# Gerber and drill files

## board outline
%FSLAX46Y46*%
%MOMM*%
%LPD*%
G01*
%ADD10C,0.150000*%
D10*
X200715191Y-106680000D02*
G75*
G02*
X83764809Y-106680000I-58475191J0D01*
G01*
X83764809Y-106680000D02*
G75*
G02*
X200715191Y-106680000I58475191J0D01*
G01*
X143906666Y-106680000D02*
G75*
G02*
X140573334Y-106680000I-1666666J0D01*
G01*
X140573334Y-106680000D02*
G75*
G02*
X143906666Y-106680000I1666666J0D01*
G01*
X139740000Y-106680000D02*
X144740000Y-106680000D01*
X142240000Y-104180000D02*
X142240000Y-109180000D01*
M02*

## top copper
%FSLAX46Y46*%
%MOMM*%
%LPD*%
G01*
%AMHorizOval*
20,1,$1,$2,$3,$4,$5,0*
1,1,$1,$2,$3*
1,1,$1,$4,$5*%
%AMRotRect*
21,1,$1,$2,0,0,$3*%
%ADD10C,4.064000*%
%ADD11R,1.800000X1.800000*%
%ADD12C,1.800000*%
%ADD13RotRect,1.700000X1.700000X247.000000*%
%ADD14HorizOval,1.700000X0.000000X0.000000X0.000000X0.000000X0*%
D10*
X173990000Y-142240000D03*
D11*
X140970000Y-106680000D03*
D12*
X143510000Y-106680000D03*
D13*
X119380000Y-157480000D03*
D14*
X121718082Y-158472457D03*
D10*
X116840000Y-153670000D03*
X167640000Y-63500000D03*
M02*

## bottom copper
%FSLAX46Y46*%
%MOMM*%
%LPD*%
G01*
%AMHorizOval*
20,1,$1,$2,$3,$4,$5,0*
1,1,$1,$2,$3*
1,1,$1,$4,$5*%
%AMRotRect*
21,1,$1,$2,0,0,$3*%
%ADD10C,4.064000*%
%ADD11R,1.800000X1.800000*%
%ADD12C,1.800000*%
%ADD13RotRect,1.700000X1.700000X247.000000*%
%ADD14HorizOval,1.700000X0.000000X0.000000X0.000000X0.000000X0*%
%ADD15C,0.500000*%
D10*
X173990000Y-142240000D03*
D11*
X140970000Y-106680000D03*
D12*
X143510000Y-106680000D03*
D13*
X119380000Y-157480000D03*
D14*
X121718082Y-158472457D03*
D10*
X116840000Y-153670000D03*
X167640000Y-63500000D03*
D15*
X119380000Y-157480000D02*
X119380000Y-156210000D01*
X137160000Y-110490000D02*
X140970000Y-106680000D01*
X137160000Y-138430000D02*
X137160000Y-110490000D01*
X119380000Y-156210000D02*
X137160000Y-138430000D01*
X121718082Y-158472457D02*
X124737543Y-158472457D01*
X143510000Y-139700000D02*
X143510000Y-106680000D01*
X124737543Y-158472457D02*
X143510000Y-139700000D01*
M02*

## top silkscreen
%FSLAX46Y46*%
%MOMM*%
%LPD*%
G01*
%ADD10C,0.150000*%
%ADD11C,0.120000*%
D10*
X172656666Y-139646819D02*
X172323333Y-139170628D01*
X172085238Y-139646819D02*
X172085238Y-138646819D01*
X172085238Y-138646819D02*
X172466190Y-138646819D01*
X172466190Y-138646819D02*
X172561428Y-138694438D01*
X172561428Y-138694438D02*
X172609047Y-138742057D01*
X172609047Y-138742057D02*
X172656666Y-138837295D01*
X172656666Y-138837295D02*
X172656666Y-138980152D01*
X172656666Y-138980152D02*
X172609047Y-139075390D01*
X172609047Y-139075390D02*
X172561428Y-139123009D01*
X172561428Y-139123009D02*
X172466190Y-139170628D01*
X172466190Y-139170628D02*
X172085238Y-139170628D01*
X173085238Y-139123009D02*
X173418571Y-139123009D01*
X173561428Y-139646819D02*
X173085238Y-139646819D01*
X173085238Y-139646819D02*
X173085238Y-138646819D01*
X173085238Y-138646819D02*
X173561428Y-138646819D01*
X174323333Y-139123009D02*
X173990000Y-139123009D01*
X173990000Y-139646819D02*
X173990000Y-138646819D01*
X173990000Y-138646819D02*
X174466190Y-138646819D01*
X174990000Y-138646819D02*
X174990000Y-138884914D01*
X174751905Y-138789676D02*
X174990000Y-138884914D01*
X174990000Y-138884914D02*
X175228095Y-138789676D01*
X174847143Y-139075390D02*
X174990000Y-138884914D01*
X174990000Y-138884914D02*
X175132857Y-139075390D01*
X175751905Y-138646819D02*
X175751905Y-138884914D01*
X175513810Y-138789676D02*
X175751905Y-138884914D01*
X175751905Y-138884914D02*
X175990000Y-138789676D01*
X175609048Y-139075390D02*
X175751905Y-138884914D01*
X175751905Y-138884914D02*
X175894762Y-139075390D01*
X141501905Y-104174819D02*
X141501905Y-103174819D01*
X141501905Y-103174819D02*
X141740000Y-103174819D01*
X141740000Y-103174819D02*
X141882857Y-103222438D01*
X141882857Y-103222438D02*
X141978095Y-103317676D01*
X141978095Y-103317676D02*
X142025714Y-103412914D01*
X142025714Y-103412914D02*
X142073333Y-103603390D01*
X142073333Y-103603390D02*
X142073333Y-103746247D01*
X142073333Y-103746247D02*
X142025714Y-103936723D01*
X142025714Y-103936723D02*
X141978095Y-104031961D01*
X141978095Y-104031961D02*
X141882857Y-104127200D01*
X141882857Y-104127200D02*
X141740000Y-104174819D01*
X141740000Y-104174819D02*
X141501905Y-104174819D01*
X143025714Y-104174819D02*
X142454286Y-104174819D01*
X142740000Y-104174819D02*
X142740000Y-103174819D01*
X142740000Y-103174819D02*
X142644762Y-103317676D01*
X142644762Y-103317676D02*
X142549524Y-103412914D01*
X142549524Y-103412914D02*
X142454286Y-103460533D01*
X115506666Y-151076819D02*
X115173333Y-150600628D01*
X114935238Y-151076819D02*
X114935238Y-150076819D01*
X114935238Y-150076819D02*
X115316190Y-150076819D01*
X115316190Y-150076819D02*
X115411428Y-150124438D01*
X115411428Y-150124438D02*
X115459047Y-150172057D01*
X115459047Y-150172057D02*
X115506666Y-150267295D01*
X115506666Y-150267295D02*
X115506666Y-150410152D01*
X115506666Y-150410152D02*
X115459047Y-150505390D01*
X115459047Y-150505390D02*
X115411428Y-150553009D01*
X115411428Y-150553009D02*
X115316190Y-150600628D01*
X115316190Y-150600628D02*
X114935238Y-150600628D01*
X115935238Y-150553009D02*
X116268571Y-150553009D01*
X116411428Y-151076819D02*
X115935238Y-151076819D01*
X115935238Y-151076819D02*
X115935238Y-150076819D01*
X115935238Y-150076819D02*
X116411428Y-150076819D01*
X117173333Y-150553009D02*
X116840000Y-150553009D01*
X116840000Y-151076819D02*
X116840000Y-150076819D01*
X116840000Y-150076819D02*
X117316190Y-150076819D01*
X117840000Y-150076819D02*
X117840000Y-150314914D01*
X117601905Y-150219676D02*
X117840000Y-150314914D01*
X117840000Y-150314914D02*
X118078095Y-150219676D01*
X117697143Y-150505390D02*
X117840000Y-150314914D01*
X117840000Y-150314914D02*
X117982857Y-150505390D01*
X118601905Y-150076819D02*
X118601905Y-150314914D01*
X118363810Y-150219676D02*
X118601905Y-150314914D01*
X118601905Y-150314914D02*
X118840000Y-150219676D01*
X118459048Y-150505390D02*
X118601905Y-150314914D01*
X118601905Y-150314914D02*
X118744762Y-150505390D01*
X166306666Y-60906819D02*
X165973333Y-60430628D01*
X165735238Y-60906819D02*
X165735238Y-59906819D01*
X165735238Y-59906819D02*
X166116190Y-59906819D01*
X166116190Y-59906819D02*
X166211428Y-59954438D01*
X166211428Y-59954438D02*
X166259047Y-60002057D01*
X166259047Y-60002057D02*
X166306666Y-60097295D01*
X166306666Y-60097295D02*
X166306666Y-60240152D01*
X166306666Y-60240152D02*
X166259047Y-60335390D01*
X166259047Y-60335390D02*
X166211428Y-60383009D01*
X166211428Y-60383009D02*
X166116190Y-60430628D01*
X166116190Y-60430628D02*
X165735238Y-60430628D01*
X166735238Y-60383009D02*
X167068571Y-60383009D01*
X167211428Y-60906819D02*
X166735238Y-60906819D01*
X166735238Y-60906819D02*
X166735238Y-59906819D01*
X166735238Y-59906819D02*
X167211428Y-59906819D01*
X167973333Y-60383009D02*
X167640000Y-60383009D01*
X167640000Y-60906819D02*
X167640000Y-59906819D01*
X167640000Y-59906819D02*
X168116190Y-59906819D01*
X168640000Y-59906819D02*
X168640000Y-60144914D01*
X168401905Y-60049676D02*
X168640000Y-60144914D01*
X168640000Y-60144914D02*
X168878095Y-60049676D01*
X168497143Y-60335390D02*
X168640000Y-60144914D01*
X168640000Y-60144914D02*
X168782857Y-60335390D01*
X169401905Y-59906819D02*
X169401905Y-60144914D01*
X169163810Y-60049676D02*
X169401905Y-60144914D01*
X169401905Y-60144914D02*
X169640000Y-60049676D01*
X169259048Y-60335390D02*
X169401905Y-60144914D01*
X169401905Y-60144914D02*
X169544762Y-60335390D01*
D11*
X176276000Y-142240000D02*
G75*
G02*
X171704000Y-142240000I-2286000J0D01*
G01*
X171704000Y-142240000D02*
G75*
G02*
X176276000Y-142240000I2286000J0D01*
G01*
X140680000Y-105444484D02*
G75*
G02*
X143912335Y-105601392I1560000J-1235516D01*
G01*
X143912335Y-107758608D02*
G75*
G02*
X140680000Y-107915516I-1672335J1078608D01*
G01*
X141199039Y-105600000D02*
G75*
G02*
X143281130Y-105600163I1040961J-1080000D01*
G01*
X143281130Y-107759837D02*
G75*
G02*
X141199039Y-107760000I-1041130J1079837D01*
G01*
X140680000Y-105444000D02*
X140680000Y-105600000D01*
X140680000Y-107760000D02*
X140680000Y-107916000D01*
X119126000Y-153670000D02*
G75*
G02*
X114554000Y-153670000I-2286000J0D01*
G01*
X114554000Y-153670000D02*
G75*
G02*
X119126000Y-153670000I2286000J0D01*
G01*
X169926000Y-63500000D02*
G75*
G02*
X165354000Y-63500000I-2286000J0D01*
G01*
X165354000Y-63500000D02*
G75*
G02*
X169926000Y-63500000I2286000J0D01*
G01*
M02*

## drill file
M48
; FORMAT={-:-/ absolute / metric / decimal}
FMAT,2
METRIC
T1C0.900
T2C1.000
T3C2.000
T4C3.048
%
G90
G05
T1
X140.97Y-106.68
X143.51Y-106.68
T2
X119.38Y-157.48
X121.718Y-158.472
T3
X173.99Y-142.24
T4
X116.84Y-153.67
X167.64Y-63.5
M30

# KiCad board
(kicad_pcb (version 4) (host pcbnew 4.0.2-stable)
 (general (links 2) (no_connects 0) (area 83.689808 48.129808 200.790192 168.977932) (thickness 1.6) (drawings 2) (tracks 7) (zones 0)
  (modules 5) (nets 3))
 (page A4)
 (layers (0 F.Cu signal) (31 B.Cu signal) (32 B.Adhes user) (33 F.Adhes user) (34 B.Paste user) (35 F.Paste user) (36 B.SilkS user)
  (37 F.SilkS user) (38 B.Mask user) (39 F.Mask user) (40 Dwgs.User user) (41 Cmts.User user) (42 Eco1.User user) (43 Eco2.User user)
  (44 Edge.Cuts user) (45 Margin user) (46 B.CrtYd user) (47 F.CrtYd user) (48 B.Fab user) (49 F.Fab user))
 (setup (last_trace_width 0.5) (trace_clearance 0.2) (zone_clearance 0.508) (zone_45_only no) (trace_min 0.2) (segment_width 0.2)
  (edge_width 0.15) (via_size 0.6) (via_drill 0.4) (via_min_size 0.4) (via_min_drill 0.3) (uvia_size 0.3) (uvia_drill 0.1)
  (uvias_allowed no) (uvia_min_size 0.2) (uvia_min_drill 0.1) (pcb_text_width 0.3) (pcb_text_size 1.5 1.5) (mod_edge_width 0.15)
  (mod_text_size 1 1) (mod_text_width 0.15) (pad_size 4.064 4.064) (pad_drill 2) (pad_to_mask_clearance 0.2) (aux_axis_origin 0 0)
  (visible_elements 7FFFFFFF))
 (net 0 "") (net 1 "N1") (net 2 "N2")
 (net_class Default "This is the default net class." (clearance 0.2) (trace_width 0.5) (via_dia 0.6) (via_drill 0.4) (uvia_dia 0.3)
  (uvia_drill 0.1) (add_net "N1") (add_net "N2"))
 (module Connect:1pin (layer F.Cu) (at 173.99 142.24)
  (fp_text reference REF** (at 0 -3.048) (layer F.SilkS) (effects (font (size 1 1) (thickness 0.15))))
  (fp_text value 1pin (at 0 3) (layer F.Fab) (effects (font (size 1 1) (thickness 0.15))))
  (fp_circle (center 0 0) (end 0 -2.286) (layer F.SilkS) (width 0.12))
  (pad 1 thru_hole circle (at 0 0) (size 4.064 4.064) (drill 2) (layers *.Cu *.Mask)))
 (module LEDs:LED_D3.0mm (layer F.Cu) (at 140.97 106.68)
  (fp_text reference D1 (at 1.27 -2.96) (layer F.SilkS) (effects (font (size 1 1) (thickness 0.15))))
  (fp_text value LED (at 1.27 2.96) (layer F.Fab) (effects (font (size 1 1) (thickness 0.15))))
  (fp_arc (start 1.27 0) (end -0.29 -1.235516) (angle 108.8) (layer F.SilkS) (width 0.12))
  (fp_arc (start 1.27 0) (end -0.29 1.235516) (angle -108.8) (layer F.SilkS) (width 0.12))
  (fp_arc (start 1.27 0) (end 0.229039 -1.08) (angle 87.9) (layer F.SilkS) (width 0.12))
  (fp_arc (start 1.27 0) (end 0.229039 1.08) (angle -87.9) (layer F.SilkS) (width 0.12))
  (fp_line (start -0.29 -1.236) (end -0.29 -1.08) (layer F.SilkS) (width 0.12))
  (fp_line (start -0.29 1.08) (end -0.29 1.236) (layer F.SilkS) (width 0.12))
  (pad 1 thru_hole rect (at 0 0) (size 1.8 1.8) (drill 0.9) (layers *.Cu *.Mask) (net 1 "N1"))
  (pad 2 thru_hole circle (at 2.54 0) (size 1.8 1.8) (drill 0.9) (layers *.Cu *.Mask) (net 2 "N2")))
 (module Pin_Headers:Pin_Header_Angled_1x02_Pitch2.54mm (layer B.Cu) (at 119.38 157.48 247)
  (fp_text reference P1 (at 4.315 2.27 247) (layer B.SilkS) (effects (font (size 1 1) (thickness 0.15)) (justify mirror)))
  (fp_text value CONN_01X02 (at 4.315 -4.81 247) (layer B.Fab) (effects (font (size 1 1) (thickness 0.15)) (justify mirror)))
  (pad 1 thru_hole rect (at 0 0 247) (size 1.7 1.7) (drill 1) (layers *.Cu *.Mask) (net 1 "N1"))
  (pad 2 thru_hole oval (at 0 -2.54 247) (size 1.7 1.7) (drill 1) (layers *.Cu *.Mask) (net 2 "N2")))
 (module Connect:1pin (layer F.Cu) (at 116.84 153.67)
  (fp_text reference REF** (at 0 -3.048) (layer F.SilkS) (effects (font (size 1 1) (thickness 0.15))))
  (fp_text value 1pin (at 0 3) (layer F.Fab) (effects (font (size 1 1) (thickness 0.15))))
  (fp_circle (center 0 0) (end 0 -2.286) (layer F.SilkS) (width 0.12))
  (pad 1 thru_hole circle (at 0 0) (size 4.064 4.064) (drill 3.048) (layers *.Cu *.Mask)))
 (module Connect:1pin (layer F.Cu) (at 167.64 63.5)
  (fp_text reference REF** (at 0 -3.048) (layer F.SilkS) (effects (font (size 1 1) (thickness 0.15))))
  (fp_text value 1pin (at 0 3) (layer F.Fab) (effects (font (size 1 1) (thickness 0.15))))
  (fp_circle (center 0 0) (end 0 -2.286) (layer F.SilkS) (width 0.12))
  (pad 1 thru_hole circle (at 0 0) (size 4.064 4.064) (drill 3.048) (layers *.Cu *.Mask)))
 (gr_circle (center 142.24 106.68) (end 190.5 139.7) (layer Edge.Cuts) (width 0.15))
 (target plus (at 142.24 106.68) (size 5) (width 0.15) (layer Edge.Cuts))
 (segment (start 119.38 157.48) (end 119.38 156.21) (width 0.5) (layer B.Cu) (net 1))
 (segment (start 137.16 110.49) (end 140.97 106.68) (width 0.5) (layer B.Cu) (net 1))
 (segment (start 137.16 138.43) (end 137.16 110.49) (width 0.5) (layer B.Cu) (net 1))
 (segment (start 119.38 156.21) (end 137.16 138.43) (width 0.5) (layer B.Cu) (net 1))
 (segment (start 121.718082 158.472457) (end 124.737543 158.472457) (width 0.5) (layer B.Cu) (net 2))
 (segment (start 143.51 139.7) (end 143.51 106.68) (width 0.5) (layer B.Cu) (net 2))
 (segment (start 124.737543 158.472457) (end 143.51 139.7) (width 0.5) (layer B.Cu) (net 2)))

